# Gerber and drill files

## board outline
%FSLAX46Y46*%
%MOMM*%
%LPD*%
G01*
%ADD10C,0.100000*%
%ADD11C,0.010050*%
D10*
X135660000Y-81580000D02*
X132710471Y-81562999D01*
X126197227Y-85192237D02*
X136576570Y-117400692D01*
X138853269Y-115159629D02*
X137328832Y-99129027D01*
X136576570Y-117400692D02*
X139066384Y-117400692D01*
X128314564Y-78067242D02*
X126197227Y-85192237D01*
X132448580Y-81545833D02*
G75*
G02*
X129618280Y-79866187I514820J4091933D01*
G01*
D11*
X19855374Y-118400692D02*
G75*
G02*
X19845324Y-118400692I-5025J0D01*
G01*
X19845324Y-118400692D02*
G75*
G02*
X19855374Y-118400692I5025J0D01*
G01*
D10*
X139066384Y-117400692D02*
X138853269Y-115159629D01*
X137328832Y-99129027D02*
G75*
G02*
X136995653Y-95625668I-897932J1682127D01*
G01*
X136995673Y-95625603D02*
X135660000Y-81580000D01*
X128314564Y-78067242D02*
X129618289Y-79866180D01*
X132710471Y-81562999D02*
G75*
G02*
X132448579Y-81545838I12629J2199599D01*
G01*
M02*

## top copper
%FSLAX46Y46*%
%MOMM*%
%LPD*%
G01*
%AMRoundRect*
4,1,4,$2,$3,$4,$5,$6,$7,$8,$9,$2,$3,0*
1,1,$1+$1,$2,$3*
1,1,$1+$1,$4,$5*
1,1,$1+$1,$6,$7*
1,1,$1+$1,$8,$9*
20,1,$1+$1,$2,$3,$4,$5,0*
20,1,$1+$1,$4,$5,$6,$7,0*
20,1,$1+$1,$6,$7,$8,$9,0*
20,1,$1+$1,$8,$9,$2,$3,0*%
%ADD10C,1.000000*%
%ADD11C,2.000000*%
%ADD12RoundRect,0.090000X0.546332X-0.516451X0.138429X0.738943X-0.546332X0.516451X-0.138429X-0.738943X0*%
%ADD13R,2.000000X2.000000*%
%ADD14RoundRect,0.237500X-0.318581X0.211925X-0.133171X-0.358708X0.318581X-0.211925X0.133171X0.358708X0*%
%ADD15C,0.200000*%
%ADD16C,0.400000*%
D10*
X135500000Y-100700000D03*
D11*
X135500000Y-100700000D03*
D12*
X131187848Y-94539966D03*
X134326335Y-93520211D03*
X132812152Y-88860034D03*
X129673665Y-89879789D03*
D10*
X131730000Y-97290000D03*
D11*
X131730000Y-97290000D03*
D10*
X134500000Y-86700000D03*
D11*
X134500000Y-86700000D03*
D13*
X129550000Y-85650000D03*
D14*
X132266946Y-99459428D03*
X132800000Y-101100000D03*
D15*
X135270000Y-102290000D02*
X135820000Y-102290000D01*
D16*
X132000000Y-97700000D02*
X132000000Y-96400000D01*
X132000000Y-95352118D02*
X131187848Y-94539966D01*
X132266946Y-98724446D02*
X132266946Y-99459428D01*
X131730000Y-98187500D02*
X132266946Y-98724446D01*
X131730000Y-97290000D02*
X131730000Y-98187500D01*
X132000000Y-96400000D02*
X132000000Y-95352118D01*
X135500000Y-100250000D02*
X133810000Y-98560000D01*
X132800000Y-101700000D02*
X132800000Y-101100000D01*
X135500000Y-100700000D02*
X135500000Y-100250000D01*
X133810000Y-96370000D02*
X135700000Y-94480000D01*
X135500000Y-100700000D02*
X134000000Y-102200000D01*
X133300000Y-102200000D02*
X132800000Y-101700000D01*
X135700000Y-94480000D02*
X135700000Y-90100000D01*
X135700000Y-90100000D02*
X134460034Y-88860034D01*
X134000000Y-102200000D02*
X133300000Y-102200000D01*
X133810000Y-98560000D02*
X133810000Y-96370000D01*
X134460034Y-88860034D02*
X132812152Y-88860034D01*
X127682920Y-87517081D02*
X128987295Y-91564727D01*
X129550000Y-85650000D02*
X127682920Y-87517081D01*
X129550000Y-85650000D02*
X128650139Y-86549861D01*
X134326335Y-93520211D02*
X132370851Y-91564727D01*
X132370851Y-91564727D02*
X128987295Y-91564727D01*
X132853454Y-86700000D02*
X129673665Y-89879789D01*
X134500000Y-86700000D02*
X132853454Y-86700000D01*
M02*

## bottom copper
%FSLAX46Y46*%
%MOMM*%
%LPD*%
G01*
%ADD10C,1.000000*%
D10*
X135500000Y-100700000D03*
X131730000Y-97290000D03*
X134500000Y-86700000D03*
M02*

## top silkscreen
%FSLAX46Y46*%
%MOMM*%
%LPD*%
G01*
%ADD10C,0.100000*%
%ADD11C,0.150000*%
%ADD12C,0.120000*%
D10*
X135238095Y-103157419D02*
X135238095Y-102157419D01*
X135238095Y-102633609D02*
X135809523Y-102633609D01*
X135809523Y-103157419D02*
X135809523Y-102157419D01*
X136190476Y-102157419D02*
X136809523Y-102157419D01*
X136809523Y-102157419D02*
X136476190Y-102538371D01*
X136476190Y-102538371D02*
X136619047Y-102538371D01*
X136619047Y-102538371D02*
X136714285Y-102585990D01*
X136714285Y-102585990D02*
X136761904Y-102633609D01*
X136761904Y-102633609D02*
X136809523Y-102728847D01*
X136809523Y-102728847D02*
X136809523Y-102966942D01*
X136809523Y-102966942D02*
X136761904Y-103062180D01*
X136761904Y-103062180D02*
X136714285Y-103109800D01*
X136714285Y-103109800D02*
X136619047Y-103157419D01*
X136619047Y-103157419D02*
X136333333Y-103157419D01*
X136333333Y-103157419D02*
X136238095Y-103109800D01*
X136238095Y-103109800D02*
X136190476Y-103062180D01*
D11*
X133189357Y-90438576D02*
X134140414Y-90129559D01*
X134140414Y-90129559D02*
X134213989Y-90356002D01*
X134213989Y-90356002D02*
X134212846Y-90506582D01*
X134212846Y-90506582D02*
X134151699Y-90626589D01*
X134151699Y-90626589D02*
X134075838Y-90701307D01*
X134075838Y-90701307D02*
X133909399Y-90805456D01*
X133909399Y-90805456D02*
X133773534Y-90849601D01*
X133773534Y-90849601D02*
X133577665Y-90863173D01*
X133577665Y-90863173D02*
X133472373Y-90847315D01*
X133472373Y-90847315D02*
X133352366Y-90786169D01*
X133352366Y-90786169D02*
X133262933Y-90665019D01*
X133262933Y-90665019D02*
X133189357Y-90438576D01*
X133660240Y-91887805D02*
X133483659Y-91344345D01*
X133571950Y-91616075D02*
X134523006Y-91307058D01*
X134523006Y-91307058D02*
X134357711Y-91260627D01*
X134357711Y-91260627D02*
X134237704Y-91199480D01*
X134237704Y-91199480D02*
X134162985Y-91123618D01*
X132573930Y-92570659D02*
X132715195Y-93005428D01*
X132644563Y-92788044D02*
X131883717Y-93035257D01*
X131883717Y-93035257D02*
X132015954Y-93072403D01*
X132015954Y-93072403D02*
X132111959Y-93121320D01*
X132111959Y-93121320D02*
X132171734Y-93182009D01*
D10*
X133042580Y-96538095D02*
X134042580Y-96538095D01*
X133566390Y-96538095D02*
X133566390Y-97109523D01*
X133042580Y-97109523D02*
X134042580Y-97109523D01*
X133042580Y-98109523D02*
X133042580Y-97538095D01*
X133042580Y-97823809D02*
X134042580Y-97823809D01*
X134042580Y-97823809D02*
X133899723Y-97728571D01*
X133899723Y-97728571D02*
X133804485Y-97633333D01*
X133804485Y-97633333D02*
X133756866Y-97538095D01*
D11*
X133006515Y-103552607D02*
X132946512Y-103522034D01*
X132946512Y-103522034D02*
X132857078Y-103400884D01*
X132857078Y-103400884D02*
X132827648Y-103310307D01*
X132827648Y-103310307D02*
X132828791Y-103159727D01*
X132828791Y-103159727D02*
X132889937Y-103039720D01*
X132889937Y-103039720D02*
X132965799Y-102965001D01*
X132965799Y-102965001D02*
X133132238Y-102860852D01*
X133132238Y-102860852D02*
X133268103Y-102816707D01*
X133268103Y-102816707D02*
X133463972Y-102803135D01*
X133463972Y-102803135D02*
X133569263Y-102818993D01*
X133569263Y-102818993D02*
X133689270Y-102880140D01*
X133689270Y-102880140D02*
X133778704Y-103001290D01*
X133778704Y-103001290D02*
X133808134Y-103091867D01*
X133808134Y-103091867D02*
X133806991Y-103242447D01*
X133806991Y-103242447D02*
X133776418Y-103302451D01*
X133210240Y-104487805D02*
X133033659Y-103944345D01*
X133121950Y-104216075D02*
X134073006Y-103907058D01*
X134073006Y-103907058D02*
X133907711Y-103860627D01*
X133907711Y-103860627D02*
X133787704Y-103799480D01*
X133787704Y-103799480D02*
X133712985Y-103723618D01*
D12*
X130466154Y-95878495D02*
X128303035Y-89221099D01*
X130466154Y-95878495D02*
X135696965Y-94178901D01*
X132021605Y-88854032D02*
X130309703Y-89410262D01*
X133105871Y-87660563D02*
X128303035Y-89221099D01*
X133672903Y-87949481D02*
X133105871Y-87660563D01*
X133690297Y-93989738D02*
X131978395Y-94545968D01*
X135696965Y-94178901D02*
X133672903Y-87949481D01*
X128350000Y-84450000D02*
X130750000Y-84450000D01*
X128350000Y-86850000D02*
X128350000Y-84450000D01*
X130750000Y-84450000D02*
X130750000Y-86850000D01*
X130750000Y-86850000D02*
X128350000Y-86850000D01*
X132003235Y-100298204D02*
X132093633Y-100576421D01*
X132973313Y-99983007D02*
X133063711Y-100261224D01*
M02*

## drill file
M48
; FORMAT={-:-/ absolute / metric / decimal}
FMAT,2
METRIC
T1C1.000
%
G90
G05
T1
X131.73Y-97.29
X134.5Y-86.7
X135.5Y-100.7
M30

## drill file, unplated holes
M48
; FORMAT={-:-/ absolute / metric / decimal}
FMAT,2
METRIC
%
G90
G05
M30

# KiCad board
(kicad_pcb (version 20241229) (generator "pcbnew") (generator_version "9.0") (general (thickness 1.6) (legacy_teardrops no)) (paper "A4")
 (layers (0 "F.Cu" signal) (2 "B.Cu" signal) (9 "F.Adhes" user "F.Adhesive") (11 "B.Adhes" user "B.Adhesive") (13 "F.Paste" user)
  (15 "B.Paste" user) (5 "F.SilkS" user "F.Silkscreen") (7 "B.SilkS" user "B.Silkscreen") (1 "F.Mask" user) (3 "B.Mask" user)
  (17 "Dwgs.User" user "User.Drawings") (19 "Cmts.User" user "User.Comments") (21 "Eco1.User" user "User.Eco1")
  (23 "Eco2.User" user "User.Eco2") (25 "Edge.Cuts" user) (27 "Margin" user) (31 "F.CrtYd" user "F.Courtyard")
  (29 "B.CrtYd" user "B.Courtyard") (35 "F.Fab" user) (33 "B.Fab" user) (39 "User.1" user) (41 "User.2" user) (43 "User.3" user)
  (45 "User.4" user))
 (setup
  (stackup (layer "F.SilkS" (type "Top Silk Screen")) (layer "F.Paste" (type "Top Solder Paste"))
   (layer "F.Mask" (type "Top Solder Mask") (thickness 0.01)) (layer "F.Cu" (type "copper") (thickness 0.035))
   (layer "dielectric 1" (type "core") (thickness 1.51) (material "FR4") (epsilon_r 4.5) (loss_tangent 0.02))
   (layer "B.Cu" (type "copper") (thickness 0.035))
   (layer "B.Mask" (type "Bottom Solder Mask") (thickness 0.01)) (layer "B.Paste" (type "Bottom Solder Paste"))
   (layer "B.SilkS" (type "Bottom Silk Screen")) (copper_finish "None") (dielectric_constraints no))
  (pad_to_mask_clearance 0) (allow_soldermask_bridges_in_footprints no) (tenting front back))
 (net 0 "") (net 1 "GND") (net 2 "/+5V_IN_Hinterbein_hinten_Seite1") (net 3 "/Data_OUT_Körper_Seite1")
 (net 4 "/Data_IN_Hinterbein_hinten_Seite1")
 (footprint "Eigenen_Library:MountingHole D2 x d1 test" (layer "F.Cu") (at 135.5 100.7)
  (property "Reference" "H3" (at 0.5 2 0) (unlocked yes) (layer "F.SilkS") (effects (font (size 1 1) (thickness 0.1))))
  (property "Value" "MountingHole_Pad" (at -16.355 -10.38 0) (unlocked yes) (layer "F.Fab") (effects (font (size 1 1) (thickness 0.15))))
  (pad "1" thru_hole circle (at 0 0) (size 1 1) (drill 1) (layers "*.Cu" "*.Mask") (remove_unused_layers no) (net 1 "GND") (zone_connect 2))
  (pad "1" connect circle (at 0 0) (size 2 2) (layers "F.Cu" "F.Mask") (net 1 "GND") (zone_connect 2)))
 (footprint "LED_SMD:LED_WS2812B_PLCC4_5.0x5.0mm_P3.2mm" (layer "F.Cu") (at 132 91.7 108)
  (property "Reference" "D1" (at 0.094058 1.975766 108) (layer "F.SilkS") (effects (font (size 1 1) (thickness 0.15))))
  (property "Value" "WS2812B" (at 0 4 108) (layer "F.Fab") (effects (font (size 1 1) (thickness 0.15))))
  (fp_line (start -3.5 -2.75) (end 3.5 -2.75) (stroke (width 0.12) (type solid)) (layer "F.SilkS"))
  (fp_line (start -3.5 -2.75) (end -3.5 2.75) (stroke (width 0.12) (type default)) (layer "F.SilkS"))
  (fp_line (start 2.7 0.9) (end 2.700001 -0.9) (stroke (width 0.12) (type default)) (layer "F.SilkS"))
  (fp_line (start 3.5 2.300001) (end 3.5 -2.75) (stroke (width 0.12) (type default)) (layer "F.SilkS"))
  (fp_line (start 3.05 2.749999) (end 3.5 2.300001) (stroke (width 0.12) (type default)) (layer "F.SilkS"))
  (fp_line (start -2.700001 0.9) (end -2.7 -0.9) (stroke (width 0.12) (type default)) (layer "F.SilkS"))
  (fp_line (start -3.5 2.75) (end 3.05 2.749999) (stroke (width 0.12) (type solid)) (layer "F.SilkS"))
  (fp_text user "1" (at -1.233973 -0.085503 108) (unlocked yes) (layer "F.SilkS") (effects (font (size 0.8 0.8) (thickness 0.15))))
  (pad "1" smd roundrect (at -2.449999 -1.65 108) (size 1.5 0.9) (layers "F.Cu" "F.Mask" "F.Paste") (roundrect_rratio 0.1)
   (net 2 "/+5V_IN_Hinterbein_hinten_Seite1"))
  (pad "2" smd roundrect (at -2.450001 1.65 108) (size 1.5 0.9) (layers "F.Cu" "F.Mask" "F.Paste") (roundrect_rratio 0.1)
   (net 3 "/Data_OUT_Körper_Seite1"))
  (pad "3" smd roundrect (at 2.449999 1.65 108) (size 1.5 0.9) (layers "F.Cu" "F.Mask" "F.Paste") (roundrect_rratio 0.1) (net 1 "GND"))
  (pad "4" smd roundrect (at 2.450001 -1.65 108) (size 1.5 0.9) (layers "F.Cu" "F.Mask" "F.Paste") (roundrect_rratio 0.1)
   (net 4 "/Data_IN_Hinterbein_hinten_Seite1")))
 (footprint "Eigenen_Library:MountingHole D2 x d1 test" (layer "F.Cu") (at 131.73 97.29)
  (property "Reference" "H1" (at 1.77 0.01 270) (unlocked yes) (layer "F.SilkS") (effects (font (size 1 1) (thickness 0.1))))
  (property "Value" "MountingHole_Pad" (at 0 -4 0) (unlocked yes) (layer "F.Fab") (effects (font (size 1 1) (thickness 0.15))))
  (pad "1" thru_hole circle (at 0 0) (size 1 1) (drill 1) (layers "*.Cu" "*.Mask") (remove_unused_layers no)
   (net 2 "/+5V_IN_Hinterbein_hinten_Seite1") (zone_connect 2))
  (pad "1" connect circle (at 0 0) (size 2 2) (layers "F.Cu" "F.Mask") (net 2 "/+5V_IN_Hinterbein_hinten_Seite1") (zone_connect 2)))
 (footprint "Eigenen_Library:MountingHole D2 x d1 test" (layer "F.Cu") (at 134.5 86.7)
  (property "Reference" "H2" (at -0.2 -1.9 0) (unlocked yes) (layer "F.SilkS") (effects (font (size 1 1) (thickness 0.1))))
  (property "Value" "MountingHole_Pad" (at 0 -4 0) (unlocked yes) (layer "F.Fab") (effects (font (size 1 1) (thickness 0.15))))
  (pad "1" thru_hole circle (at 0 0) (size 1 1) (drill 1) (layers "*.Cu" "*.Mask") (remove_unused_layers no)
   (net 4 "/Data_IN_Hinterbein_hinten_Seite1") (zone_connect 2))
  (pad "1" connect circle (at 0 0) (size 2 2) (layers "F.Cu" "F.Mask") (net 4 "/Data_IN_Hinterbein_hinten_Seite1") (zone_connect 2)))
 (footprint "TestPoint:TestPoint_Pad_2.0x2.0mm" (layer "F.Cu") (at 129.55 85.65)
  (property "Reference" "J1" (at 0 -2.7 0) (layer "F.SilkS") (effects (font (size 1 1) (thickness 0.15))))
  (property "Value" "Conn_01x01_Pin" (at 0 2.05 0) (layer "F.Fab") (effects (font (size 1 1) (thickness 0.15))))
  (fp_line (start -1.2 -1.2) (end 1.2 -1.2) (stroke (width 0.12) (type solid)) (layer "F.SilkS"))
  (fp_line (start -1.2 1.2) (end -1.2 -1.2) (stroke (width 0.12) (type solid)) (layer "F.SilkS"))
  (fp_line (start 1.2 -1.2) (end 1.2 1.2) (stroke (width 0.12) (type solid)) (layer "F.SilkS"))
  (fp_line (start 1.2 1.2) (end -1.2 1.2) (stroke (width 0.12) (type solid)) (layer "F.SilkS"))
  (pad "1" smd rect (at 0 0) (size 2 2) (layers "F.Cu" "F.Mask") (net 3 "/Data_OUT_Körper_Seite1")))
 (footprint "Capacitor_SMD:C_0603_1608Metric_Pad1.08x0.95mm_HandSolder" (layer "F.Cu") (at 132.533473 100.279714 -72)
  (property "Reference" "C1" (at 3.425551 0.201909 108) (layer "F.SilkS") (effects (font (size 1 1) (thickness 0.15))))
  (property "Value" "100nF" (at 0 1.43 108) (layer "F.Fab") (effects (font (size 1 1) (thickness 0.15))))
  (fp_line (start -0.146268 0.51) (end 0.146267 0.51) (stroke (width 0.12) (type solid)) (layer "F.SilkS"))
  (fp_line (start -0.146267 -0.51) (end 0.146268 -0.51) (stroke (width 0.12) (type solid)) (layer "F.SilkS"))
  (pad "1" smd roundrect (at -0.8625 0 288) (size 1.075 0.95) (layers "F.Cu" "F.Mask" "F.Paste") (roundrect_rratio 0.25)
   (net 2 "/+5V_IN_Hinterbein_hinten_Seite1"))
  (pad "2" smd roundrect (at 0.8625 0 288) (size 1.075 0.95) (layers "F.Cu" "F.Mask" "F.Paste") (roundrect_rratio 0.25) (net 1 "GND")))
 (gr_line (start 135.66 81.58) (end 132.710471 81.562999) (stroke (width 0.1) (type default)) (locked yes) (layer "Edge.Cuts"))
 (gr_line (start 126.197227 85.192237) (end 136.57657 117.400692) (stroke (width 0.1) (type default)) (locked yes) (layer "Edge.Cuts"))
 (gr_line (start 138.853269 115.159629) (end 137.328832 99.129027) (stroke (width 0.1) (type default)) (locked yes) (layer "Edge.Cuts"))
 (gr_line (start 136.57657 117.400692) (end 139.066384 117.400692) (stroke (width 0.1) (type default)) (locked yes) (layer "Edge.Cuts"))
 (gr_line (start 128.314564 78.067242) (end 126.197227 85.192237) (stroke (width 0.1) (type default)) (locked yes) (layer "Edge.Cuts"))
 (gr_arc (start 132.44858 81.545833) (mid 130.858629 81.000567) (end 129.618289 79.86618) (stroke (width 0.1) (type default)) (locked yes)
  (layer "Edge.Cuts"))
 (gr_circle (center 19.850349 118.400692) (end 19.860349 118.400692) (stroke (width 0.0001) (type default)) (fill yes) (locked yes)
  (layer "Edge.Cuts"))
 (gr_line (start 139.066384 117.400692) (end 138.853269 115.159629) (stroke (width 0.1) (type default)) (locked yes) (layer "Edge.Cuts"))
 (gr_arc (start 137.328832 99.129027) (mid 134.532637 97.627368) (end 136.995673 95.625603) (stroke (width 0.1) (type default)) (locked yes)
  (layer "Edge.Cuts"))
 (gr_line (start 136.995673 95.625603) (end 135.66 81.58) (stroke (width 0.1) (type default)) (locked yes) (layer "Edge.Cuts"))
 (gr_line (start 128.314564 78.067242) (end 129.618289 79.86618) (stroke (width 0.1) (type default)) (locked yes) (layer "Edge.Cuts"))
 (gr_arc (start 132.710471 81.562999) (mid 132.579276 81.558326) (end 132.44858 81.545833) (stroke (width 0.1) (type default)) (locked yes)
  (layer "Edge.Cuts"))
 (segment (start 135.27 102.29) (end 135.82 102.29) (width 0.2) (layer "F.Cu") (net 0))
 (segment (start 132 97.7) (end 132 96.4) (width 0.4) (layer "F.Cu") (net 2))
 (segment (start 132 95.352118) (end 131.187848 94.539966) (width 0.4) (layer "F.Cu") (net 2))
 (segment (start 132.266946 98.724446) (end 132.266946 99.459428) (width 0.4) (layer "F.Cu") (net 2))
 (segment (start 131.73 98.1875) (end 132.266946 98.724446) (width 0.4) (layer "F.Cu") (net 2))
 (segment (start 131.73 97.29) (end 131.73 98.1875) (width 0.4) (layer "F.Cu") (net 2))
 (segment (start 132 96.4) (end 132 95.352118) (width 0.4) (layer "F.Cu") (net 2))
 (segment (start 135.5 100.25) (end 133.81 98.56) (width 0.4) (layer "F.Cu") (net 1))
 (segment (start 132.8 101.7) (end 132.8 101.1) (width 0.4) (layer "F.Cu") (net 1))
 (segment (start 135.5 100.7) (end 135.5 100.25) (width 0.4) (layer "F.Cu") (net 1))
 (segment (start 133.81 96.37) (end 135.7 94.48) (width 0.4) (layer "F.Cu") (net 1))
 (segment (start 135.5 100.7) (end 134 102.2) (width 0.4) (layer "F.Cu") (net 1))
 (segment (start 133.3 102.2) (end 132.8 101.7) (width 0.4) (layer "F.Cu") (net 1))
 (segment (start 135.7 94.48) (end 135.7 90.1) (width 0.4) (layer "F.Cu") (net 1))
 (segment (start 135.7 90.1) (end 134.460034 88.860034) (width 0.4) (layer "F.Cu") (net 1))
 (segment (start 134 102.2) (end 133.3 102.2) (width 0.4) (layer "F.Cu") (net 1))
 (segment (start 133.81 98.56) (end 133.81 96.37) (width 0.4) (layer "F.Cu") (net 1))
 (segment (start 134.460034 88.860034) (end 132.812152 88.860034) (width 0.4) (layer "F.Cu") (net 1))
 (segment (start 127.68292 87.517081) (end 128.987295 91.564727) (width 0.4) (layer "F.Cu") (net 3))
 (segment (start 129.55 85.65) (end 127.68292 87.517081) (width 0.4) (layer "F.Cu") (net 3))
 (segment (start 129.55 85.65) (end 128.650139 86.549861) (width 0.4) (layer "F.Cu") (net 3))
 (segment (start 134.326335 93.520211) (end 132.370851 91.564727) (width 0.4) (layer "F.Cu") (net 3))
 (segment (start 132.370851 91.564727) (end 128.987295 91.564727) (width 0.4) (layer "F.Cu") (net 3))
 (segment (start 132.853454 86.7) (end 129.673665 89.879789) (width 0.4) (layer "F.Cu") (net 4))
 (segment (start 134.5 86.7) (end 132.853454 86.7) (width 0.4) (layer "F.Cu") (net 4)))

